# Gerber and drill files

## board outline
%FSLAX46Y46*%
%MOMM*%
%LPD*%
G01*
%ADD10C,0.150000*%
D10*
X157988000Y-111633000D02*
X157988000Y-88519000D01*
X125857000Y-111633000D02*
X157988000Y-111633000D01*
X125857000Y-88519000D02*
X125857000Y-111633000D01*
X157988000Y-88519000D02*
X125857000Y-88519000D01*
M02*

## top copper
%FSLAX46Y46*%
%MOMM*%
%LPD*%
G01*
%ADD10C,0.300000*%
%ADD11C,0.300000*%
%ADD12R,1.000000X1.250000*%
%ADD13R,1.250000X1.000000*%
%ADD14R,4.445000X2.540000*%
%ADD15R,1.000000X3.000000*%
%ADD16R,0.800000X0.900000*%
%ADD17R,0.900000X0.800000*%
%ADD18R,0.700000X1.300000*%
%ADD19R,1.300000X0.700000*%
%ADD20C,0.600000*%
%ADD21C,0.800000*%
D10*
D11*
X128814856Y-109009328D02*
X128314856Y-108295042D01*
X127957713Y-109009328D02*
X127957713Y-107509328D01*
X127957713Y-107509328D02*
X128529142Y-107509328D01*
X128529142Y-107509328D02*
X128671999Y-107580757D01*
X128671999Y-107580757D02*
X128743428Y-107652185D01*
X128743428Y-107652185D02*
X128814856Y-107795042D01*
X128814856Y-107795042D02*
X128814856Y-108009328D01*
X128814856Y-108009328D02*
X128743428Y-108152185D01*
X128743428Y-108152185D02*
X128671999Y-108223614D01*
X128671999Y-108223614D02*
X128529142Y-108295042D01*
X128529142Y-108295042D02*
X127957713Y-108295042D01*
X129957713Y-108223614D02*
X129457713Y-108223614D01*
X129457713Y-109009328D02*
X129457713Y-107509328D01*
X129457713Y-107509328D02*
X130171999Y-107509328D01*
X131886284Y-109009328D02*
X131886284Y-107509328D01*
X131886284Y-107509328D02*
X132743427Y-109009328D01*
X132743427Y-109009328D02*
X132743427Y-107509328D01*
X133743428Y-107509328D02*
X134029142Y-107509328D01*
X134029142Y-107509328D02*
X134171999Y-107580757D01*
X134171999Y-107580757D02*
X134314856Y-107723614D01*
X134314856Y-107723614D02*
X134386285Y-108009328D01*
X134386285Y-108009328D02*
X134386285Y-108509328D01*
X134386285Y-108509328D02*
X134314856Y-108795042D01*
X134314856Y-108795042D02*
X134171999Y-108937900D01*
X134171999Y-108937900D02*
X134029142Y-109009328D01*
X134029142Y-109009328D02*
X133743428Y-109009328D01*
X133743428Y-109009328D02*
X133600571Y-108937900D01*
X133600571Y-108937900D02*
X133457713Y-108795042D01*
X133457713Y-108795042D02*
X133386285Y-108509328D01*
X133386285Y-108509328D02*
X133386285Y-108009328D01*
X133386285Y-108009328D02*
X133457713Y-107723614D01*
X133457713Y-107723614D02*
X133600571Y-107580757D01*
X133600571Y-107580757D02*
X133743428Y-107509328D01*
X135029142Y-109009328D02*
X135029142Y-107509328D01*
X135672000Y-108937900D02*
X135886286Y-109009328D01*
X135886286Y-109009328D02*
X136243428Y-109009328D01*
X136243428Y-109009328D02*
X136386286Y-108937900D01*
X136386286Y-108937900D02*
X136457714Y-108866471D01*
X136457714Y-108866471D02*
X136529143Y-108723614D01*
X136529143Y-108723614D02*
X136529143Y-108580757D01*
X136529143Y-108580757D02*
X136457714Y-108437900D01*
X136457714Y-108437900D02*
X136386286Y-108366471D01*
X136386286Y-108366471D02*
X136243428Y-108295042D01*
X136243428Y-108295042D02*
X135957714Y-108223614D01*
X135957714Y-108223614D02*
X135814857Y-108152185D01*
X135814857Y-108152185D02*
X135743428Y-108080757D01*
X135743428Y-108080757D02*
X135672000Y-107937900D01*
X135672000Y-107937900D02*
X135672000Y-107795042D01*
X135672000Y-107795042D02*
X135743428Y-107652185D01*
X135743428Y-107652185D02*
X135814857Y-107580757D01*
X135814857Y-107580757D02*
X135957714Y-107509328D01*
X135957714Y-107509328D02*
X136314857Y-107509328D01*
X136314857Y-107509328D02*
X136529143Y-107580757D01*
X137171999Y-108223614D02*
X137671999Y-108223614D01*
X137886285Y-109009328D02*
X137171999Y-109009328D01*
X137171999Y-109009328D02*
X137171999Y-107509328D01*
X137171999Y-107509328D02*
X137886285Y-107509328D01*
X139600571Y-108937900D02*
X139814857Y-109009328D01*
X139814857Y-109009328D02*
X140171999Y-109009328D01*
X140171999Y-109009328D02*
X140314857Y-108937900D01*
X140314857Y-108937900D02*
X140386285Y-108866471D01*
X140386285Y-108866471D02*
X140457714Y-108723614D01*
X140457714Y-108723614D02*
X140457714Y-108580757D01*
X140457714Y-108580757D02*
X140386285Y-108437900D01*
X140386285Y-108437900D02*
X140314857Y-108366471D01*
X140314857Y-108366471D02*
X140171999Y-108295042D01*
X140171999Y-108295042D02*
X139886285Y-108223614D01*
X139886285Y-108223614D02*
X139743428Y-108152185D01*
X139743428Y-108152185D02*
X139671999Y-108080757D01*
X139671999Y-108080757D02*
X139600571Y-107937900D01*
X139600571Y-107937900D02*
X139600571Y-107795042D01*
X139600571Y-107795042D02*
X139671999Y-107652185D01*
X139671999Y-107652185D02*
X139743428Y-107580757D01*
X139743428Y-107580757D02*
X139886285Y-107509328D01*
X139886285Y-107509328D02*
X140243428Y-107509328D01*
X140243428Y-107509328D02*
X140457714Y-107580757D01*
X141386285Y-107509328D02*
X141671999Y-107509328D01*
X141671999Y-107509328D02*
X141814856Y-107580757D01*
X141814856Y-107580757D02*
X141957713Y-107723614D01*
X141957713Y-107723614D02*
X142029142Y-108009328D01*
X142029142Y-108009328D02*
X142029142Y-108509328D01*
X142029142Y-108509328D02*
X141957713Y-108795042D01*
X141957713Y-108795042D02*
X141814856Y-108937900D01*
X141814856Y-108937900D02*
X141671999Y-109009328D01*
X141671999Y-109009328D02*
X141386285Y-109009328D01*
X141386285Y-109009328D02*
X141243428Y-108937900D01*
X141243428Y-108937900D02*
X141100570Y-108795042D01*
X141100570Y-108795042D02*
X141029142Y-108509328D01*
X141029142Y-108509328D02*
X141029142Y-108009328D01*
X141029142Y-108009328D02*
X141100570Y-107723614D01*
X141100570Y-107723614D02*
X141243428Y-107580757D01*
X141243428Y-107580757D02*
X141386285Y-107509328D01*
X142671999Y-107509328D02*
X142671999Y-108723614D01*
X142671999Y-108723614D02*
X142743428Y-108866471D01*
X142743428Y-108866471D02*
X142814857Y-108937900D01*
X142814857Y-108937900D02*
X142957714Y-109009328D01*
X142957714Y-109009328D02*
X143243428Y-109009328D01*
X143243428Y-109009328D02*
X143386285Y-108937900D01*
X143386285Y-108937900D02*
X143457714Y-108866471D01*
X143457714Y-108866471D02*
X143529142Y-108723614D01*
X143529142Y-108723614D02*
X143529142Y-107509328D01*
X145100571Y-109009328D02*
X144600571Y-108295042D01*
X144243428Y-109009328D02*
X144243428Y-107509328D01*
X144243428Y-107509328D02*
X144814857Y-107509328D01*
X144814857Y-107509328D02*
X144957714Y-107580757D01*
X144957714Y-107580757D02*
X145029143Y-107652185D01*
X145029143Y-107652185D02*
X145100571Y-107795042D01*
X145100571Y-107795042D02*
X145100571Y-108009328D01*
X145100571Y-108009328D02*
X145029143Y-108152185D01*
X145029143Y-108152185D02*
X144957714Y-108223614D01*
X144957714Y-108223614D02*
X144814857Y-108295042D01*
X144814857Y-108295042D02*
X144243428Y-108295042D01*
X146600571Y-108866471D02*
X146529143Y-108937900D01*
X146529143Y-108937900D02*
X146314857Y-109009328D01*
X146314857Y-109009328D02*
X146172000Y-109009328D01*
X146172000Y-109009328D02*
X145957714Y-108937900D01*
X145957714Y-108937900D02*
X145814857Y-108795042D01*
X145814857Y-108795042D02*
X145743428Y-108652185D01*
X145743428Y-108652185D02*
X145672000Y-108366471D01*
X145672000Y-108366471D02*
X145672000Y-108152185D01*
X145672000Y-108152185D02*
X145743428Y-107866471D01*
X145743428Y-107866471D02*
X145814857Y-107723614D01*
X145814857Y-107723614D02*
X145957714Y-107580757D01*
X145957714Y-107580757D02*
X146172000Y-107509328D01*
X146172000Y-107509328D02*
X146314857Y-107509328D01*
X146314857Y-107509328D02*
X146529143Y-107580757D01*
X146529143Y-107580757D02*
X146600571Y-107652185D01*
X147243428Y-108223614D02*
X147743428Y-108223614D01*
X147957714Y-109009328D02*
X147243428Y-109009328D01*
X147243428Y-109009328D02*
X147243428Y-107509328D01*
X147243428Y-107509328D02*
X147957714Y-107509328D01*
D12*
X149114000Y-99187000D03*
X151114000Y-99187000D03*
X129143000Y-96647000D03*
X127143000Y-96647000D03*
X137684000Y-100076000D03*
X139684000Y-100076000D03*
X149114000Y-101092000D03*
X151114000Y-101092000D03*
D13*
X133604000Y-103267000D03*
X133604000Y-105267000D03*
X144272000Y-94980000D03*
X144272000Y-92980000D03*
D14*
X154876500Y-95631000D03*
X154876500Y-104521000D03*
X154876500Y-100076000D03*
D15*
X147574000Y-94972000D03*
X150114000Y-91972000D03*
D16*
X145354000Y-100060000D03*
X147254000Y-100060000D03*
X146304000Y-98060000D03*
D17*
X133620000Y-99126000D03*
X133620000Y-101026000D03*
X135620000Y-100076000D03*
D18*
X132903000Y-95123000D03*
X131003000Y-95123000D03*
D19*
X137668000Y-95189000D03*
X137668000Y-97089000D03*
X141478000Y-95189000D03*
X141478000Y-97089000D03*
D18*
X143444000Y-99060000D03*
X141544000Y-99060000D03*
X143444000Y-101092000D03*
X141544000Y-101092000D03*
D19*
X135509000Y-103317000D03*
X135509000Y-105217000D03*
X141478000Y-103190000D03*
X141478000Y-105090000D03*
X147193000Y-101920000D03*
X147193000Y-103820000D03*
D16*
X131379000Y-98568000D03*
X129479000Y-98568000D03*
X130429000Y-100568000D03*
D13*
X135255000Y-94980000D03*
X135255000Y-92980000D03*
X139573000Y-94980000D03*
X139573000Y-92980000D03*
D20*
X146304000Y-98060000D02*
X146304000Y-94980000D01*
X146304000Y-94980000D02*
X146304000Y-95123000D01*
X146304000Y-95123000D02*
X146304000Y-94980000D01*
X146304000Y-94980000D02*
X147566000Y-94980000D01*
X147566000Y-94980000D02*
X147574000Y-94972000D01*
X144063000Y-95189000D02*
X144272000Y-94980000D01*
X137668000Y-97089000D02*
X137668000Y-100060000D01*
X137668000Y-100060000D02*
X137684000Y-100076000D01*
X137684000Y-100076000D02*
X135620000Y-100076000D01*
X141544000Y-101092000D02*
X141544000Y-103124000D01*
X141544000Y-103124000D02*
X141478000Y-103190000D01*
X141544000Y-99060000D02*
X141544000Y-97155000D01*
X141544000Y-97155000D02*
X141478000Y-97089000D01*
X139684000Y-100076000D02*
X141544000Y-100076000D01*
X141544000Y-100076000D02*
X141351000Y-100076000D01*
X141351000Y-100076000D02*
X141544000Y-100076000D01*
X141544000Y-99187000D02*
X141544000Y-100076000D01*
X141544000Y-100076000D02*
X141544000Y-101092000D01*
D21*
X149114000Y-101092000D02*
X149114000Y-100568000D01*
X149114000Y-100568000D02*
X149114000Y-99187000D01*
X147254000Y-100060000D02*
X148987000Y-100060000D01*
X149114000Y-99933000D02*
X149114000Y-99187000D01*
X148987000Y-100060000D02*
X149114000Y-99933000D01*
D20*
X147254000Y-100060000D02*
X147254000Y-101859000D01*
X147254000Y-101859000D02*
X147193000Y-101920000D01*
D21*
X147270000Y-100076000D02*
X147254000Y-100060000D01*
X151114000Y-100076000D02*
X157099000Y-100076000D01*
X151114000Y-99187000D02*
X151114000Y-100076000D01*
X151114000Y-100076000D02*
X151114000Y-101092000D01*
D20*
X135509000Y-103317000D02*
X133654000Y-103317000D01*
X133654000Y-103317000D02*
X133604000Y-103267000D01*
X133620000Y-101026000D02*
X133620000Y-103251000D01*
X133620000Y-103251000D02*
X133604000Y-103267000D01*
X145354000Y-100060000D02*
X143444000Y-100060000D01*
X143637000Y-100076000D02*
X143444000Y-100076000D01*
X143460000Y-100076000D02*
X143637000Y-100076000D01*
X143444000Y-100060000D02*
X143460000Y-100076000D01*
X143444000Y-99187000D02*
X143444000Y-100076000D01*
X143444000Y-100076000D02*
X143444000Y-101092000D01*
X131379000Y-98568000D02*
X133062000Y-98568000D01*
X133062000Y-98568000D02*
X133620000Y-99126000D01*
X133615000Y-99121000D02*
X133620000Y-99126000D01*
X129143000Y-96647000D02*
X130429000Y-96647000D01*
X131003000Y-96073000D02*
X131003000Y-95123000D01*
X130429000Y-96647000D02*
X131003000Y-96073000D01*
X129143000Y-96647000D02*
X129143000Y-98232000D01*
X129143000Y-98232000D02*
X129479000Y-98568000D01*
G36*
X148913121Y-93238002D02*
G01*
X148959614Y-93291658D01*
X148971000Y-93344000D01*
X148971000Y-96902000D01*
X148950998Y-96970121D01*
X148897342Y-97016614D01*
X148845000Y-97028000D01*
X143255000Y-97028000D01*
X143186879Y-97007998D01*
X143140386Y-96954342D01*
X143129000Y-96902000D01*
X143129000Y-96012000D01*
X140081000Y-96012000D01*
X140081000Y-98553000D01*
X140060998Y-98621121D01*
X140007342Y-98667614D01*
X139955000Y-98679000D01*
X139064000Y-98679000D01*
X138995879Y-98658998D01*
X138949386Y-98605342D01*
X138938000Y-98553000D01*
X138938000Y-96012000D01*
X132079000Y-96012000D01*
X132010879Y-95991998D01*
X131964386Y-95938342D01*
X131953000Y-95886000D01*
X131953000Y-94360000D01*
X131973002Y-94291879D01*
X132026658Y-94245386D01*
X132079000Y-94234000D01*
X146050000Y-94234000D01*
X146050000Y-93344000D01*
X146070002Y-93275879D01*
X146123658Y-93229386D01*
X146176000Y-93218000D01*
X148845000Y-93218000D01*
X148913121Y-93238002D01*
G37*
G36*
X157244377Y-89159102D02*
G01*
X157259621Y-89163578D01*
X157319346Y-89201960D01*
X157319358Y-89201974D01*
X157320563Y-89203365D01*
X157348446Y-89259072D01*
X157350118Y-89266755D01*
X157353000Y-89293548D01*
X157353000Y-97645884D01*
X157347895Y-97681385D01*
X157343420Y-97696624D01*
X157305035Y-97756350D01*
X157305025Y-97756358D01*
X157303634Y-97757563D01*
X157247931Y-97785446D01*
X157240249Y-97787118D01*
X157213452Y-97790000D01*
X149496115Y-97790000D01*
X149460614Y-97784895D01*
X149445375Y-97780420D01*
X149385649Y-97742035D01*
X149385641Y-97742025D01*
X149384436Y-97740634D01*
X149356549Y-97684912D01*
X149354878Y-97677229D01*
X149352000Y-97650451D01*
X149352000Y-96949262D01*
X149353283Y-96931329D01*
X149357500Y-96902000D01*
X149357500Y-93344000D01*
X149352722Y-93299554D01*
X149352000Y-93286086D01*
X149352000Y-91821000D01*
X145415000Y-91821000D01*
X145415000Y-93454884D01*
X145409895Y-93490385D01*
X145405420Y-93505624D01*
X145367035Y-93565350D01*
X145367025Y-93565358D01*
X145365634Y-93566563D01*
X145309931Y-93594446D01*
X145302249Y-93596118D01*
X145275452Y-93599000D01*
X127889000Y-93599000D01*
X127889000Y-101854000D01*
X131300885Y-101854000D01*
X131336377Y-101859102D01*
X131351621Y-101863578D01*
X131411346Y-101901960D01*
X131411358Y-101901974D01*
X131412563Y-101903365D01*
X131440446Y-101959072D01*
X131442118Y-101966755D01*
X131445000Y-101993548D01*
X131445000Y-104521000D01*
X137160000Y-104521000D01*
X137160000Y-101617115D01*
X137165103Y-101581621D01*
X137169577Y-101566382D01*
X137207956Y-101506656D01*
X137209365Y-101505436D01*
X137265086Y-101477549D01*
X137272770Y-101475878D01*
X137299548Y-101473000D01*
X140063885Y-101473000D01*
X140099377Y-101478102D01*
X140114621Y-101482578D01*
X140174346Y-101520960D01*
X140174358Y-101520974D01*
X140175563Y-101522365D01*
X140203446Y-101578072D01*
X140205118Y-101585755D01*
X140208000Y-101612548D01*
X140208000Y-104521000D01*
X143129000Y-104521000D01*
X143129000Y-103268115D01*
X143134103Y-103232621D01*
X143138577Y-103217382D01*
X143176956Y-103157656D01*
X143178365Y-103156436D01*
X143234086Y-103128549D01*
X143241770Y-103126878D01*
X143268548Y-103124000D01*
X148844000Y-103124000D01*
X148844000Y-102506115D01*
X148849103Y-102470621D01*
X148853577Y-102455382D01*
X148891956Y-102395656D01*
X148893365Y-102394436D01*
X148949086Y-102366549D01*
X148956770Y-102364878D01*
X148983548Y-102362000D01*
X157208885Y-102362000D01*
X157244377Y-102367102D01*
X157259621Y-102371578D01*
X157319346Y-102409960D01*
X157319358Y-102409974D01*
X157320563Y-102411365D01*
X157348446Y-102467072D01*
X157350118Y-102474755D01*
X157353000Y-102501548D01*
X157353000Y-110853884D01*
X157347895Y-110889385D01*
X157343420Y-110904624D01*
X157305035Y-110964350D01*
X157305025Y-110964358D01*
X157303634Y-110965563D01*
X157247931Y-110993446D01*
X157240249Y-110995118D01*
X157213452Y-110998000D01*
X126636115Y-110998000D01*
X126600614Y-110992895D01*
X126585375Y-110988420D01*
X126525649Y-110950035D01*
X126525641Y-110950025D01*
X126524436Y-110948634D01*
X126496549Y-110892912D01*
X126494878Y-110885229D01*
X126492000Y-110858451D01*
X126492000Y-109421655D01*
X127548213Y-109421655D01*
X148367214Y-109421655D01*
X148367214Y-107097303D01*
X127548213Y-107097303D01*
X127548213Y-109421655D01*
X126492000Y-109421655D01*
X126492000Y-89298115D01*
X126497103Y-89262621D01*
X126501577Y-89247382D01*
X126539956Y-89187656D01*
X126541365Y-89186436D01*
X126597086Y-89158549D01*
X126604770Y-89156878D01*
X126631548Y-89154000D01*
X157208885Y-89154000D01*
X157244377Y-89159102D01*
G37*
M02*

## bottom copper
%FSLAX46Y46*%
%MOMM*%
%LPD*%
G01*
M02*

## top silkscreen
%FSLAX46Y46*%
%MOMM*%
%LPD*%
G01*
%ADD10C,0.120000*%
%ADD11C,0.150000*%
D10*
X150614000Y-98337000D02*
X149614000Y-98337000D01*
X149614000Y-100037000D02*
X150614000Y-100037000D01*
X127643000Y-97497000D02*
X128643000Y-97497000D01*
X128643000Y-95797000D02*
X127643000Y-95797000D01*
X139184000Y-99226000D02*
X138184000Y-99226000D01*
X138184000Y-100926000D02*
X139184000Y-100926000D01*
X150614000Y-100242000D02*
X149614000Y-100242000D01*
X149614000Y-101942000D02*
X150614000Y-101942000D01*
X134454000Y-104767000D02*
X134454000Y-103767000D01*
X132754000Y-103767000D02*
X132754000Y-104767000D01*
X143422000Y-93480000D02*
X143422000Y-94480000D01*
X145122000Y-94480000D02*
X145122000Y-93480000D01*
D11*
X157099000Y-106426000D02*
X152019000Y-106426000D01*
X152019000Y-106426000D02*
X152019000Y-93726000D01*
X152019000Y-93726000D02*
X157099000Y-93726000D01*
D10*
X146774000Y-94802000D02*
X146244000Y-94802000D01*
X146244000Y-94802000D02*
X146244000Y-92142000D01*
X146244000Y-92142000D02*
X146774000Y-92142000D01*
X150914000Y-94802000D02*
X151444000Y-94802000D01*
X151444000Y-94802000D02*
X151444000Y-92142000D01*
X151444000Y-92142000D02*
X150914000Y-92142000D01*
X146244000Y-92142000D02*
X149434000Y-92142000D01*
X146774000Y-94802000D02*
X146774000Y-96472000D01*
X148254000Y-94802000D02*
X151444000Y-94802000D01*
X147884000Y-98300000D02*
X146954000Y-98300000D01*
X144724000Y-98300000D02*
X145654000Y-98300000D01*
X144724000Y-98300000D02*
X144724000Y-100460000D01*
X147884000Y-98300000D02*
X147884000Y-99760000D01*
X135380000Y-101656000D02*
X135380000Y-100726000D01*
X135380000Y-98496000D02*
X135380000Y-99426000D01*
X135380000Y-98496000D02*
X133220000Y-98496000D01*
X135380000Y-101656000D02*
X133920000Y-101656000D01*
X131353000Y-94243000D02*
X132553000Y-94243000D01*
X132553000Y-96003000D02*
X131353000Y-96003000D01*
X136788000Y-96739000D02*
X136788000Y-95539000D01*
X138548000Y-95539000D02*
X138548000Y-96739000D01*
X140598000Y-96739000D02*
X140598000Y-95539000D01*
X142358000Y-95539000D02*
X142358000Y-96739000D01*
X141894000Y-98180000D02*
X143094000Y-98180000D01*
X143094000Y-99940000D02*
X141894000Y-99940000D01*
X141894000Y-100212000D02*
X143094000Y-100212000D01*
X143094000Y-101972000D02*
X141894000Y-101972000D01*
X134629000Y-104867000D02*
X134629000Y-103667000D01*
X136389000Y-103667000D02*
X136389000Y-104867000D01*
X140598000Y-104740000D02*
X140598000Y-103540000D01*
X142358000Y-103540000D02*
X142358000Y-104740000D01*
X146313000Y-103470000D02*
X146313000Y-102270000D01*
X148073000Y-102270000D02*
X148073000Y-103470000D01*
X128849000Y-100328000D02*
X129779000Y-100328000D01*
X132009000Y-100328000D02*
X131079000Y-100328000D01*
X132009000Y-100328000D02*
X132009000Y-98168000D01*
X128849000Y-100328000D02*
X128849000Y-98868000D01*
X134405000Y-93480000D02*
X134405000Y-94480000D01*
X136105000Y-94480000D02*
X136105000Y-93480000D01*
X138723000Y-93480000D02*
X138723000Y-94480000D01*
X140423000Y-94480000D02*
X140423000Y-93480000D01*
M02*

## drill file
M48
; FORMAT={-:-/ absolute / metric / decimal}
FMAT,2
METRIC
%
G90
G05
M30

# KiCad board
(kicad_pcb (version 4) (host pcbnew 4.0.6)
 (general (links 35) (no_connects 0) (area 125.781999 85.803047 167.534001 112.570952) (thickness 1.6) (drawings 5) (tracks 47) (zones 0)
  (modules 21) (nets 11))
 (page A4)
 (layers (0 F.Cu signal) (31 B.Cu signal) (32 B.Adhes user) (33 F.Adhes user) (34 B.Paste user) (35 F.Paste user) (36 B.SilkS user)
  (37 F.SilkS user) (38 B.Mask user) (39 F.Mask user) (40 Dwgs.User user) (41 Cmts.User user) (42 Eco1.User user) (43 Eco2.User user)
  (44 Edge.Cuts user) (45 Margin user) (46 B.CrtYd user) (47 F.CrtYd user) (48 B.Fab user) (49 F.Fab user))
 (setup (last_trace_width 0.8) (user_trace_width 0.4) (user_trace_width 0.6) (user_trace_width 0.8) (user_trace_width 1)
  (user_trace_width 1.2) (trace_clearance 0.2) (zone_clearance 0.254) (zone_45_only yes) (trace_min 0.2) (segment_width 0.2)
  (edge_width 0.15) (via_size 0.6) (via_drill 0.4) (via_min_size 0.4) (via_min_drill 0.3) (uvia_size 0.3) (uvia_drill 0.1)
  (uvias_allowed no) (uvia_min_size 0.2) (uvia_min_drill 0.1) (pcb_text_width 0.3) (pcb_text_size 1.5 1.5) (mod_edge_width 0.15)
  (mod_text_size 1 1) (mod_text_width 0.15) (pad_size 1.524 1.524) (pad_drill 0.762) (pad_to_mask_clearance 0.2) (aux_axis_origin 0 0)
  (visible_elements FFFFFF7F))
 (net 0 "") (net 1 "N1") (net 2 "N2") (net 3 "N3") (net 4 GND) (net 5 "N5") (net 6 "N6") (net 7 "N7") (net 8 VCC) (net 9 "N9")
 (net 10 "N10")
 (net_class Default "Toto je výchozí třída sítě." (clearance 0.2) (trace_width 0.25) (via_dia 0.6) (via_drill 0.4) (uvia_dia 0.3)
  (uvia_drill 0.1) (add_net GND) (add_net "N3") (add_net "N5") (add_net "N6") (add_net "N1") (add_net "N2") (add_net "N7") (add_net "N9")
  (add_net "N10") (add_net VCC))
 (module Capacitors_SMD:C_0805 (layer F.Cu) (at 150.114 99.187)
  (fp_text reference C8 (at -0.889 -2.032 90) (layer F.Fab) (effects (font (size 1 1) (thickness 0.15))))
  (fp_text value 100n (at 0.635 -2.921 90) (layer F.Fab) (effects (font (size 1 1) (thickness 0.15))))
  (fp_line (start 0.5 -0.85) (end -0.5 -0.85) (layer F.SilkS) (width 0.12))
  (fp_line (start -0.5 0.85) (end 0.5 0.85) (layer F.SilkS) (width 0.12))
  (pad 1 smd rect (at -1 0) (size 1 1.25) (layers F.Cu F.Paste F.Mask) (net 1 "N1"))
  (pad 2 smd rect (at 1 0) (size 1 1.25) (layers F.Cu F.Paste F.Mask) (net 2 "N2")))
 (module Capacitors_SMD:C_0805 (layer F.Cu) (at 128.143 96.647 180)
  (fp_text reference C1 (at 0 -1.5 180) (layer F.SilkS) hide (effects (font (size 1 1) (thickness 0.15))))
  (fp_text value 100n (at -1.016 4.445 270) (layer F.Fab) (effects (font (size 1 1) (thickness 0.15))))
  (fp_line (start 0.5 -0.85) (end -0.5 -0.85) (layer F.SilkS) (width 0.12))
  (fp_line (start -0.5 0.85) (end 0.5 0.85) (layer F.SilkS) (width 0.12))
  (pad 1 smd rect (at -1 0 180) (size 1 1.25) (layers F.Cu F.Paste F.Mask) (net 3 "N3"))
  (pad 2 smd rect (at 1 0 180) (size 1 1.25) (layers F.Cu F.Paste F.Mask) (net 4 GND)))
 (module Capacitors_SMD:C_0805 (layer F.Cu) (at 138.684 100.076)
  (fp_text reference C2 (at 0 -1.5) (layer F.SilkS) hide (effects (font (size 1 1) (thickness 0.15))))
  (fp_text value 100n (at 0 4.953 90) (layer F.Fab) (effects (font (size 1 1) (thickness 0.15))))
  (fp_line (start 0.5 -0.85) (end -0.5 -0.85) (layer F.SilkS) (width 0.12))
  (fp_line (start -0.5 0.85) (end 0.5 0.85) (layer F.SilkS) (width 0.12))
  (pad 1 smd rect (at -1 0) (size 1 1.25) (layers F.Cu F.Paste F.Mask) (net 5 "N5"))
  (pad 2 smd rect (at 1 0) (size 1 1.25) (layers F.Cu F.Paste F.Mask) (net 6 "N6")))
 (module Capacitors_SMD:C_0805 (layer F.Cu) (at 150.114 101.092)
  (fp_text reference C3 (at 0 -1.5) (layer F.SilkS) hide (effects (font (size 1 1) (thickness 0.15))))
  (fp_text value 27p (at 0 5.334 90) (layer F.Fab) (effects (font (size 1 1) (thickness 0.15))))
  (fp_line (start 0.5 -0.85) (end -0.5 -0.85) (layer F.SilkS) (width 0.12))
  (fp_line (start -0.5 0.85) (end 0.5 0.85) (layer F.SilkS) (width 0.12))
  (pad 1 smd rect (at -1 0) (size 1 1.25) (layers F.Cu F.Paste F.Mask) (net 1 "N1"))
  (pad 2 smd rect (at 1 0) (size 1 1.25) (layers F.Cu F.Paste F.Mask) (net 2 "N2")))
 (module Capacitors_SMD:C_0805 (layer F.Cu) (at 133.604 104.267 270)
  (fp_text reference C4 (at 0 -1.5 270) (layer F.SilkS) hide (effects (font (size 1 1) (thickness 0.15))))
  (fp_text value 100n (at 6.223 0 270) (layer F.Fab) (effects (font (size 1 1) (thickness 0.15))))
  (fp_line (start 0.5 -0.85) (end -0.5 -0.85) (layer F.SilkS) (width 0.12))
  (fp_line (start -0.5 0.85) (end 0.5 0.85) (layer F.SilkS) (width 0.12))
  (pad 1 smd rect (at -1 0 270) (size 1 1.25) (layers F.Cu F.Paste F.Mask) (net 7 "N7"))
  (pad 2 smd rect (at 1 0 270) (size 1 1.25) (layers F.Cu F.Paste F.Mask) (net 4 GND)))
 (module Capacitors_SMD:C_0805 (layer F.Cu) (at 144.272 93.98 90)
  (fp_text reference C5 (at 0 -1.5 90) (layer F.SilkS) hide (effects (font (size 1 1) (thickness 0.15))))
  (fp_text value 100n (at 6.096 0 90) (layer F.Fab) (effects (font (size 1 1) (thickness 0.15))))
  (fp_line (start 0.5 -0.85) (end -0.5 -0.85) (layer F.SilkS) (width 0.12))
  (fp_line (start -0.5 0.85) (end 0.5 0.85) (layer F.SilkS) (width 0.12))
  (pad 1 smd rect (at -1 0 90) (size 1 1.25) (layers F.Cu F.Paste F.Mask) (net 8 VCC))
  (pad 2 smd rect (at 1 0 90) (size 1 1.25) (layers F.Cu F.Paste F.Mask) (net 4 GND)))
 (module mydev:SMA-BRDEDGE (layer F.Cu) (at 157.099 100.076 180)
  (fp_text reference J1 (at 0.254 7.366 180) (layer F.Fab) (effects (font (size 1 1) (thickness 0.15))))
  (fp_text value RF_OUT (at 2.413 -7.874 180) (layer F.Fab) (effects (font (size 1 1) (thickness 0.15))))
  (fp_line (start 0 -6.35) (end 5.08 -6.35) (layer F.SilkS) (width 0.15))
  (fp_line (start 5.08 -6.35) (end 5.08 6.35) (layer F.SilkS) (width 0.15))
  (fp_line (start 5.08 6.35) (end 0 6.35) (layer F.SilkS) (width 0.15))
  (pad 2 smd rect (at 0 4.445 180) (size 4.445 2.54) (drill (offset 2.2225 0)) (layers F.Cu F.Paste F.Mask) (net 4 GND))
  (pad 2 smd rect (at 0 -4.445 180) (size 4.445 2.54) (drill (offset 2.2225 0)) (layers F.Cu F.Paste F.Mask) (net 4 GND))
  (pad 1 smd rect (at 0 0 180) (size 4.445 2.54) (drill (offset 2.2225 0)) (layers F.Cu F.Paste F.Mask) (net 2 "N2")))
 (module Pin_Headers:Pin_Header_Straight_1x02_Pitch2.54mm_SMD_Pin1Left (layer F.Cu) (at 148.844 93.472 90)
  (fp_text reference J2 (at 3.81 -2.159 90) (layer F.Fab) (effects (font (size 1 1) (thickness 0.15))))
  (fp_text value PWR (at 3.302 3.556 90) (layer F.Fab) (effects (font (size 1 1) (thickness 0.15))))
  (fp_line (start -1.33 -2.07) (end -1.33 -2.6) (layer F.SilkS) (width 0.12))
  (fp_line (start -1.33 -2.6) (end 1.33 -2.6) (layer F.SilkS) (width 0.12))
  (fp_line (start 1.33 -2.6) (end 1.33 -2.07) (layer F.SilkS) (width 0.12))
  (fp_line (start -1.33 2.07) (end -1.33 2.6) (layer F.SilkS) (width 0.12))
  (fp_line (start -1.33 2.6) (end 1.33 2.6) (layer F.SilkS) (width 0.12))
  (fp_line (start 1.33 2.6) (end 1.33 2.07) (layer F.SilkS) (width 0.12))
  (fp_line (start 1.33 -2.6) (end 1.33 0.59) (layer F.SilkS) (width 0.12))
  (fp_line (start -1.33 -2.07) (end -3 -2.07) (layer F.SilkS) (width 0.12))
  (fp_line (start -1.33 -0.59) (end -1.33 2.6) (layer F.SilkS) (width 0.12))
  (pad 1 smd rect (at -1.5 -1.27 90) (size 3 1) (layers F.Cu F.Mask) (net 8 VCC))
  (pad 2 smd rect (at 1.5 1.27 90) (size 3 1) (layers F.Cu F.Mask) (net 4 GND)))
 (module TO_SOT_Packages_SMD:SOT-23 (layer F.Cu) (at 146.304 99.06 90)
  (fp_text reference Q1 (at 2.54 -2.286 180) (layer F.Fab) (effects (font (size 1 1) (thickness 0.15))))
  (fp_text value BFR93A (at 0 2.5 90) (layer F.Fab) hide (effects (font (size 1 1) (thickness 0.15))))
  (fp_line (start 0.76 1.58) (end 0.76 0.65) (layer F.SilkS) (width 0.12))
  (fp_line (start 0.76 -1.58) (end 0.76 -0.65) (layer F.SilkS) (width 0.12))
  (fp_line (start 0.76 -1.58) (end -1.4 -1.58) (layer F.SilkS) (width 0.12))
  (fp_line (start 0.76 1.58) (end -0.7 1.58) (layer F.SilkS) (width 0.12))
  (pad 1 smd rect (at -1 -0.95 90) (size 0.9 0.8) (layers F.Cu F.Paste F.Mask) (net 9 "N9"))
  (pad 2 smd rect (at -1 0.95 90) (size 0.9 0.8) (layers F.Cu F.Paste F.Mask) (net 1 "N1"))
  (pad 3 smd rect (at 1 0 90) (size 0.9 0.8) (layers F.Cu F.Paste F.Mask) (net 8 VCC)))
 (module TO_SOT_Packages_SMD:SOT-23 (layer F.Cu) (at 134.62 100.076)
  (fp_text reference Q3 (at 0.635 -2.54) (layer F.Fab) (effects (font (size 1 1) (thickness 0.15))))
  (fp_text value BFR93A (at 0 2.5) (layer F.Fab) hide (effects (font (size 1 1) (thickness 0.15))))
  (fp_line (start 0.76 1.58) (end 0.76 0.65) (layer F.SilkS) (width 0.12))
  (fp_line (start 0.76 -1.58) (end 0.76 -0.65) (layer F.SilkS) (width 0.12))
  (fp_line (start 0.76 -1.58) (end -1.4 -1.58) (layer F.SilkS) (width 0.12))
  (fp_line (start 0.76 1.58) (end -0.7 1.58) (layer F.SilkS) (width 0.12))
  (pad 1 smd rect (at -1 -0.95) (size 0.9 0.8) (layers F.Cu F.Paste F.Mask) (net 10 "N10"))
  (pad 2 smd rect (at -1 0.95) (size 0.9 0.8) (layers F.Cu F.Paste F.Mask) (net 7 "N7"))
  (pad 3 smd rect (at 1 0) (size 0.9 0.8) (layers F.Cu F.Paste F.Mask) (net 5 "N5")))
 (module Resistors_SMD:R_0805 (layer F.Cu) (at 131.953 95.123 180)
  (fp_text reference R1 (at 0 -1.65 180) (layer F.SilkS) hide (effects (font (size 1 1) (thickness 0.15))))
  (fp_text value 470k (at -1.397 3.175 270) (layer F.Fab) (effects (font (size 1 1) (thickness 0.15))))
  (fp_line (start 0.6 0.88) (end -0.6 0.88) (layer F.SilkS) (width 0.12))
  (fp_line (start -0.6 -0.88) (end 0.6 -0.88) (layer F.SilkS) (width 0.12))
  (pad 1 smd rect (at -0.95 0 180) (size 0.7 1.3) (layers F.Cu F.Paste F.Mask) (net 8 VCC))
  (pad 2 smd rect (at 0.95 0 180) (size 0.7 1.3) (layers F.Cu F.Paste F.Mask) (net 3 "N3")))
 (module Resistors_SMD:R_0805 (layer F.Cu) (at 137.668 96.139 270)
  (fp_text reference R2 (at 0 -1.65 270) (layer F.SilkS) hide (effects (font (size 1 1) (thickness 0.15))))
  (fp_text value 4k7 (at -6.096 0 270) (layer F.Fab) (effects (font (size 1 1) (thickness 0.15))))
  (fp_line (start 0.6 0.88) (end -0.6 0.88) (layer F.SilkS) (width 0.12))
  (fp_line (start -0.6 -0.88) (end 0.6 -0.88) (layer F.SilkS) (width 0.12))
  (pad 1 smd rect (at -0.95 0 270) (size 0.7 1.3) (layers F.Cu F.Paste F.Mask) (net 8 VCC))
  (pad 2 smd rect (at 0.95 0 270) (size 0.7 1.3) (layers F.Cu F.Paste F.Mask) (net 5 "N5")))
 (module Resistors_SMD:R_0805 (layer F.Cu) (at 141.478 96.139 270)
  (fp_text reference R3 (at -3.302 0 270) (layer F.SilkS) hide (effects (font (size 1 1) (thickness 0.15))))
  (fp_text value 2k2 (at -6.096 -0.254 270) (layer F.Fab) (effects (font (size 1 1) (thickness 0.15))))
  (fp_line (start 0.6 0.88) (end -0.6 0.88) (layer F.SilkS) (width 0.12))
  (fp_line (start -0.6 -0.88) (end 0.6 -0.88) (layer F.SilkS) (width 0.12))
  (pad 1 smd rect (at -0.95 0 270) (size 0.7 1.3) (layers F.Cu F.Paste F.Mask) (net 8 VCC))
  (pad 2 smd rect (at 0.95 0 270) (size 0.7 1.3) (layers F.Cu F.Paste F.Mask) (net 6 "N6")))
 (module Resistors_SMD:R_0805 (layer F.Cu) (at 142.494 99.06 180)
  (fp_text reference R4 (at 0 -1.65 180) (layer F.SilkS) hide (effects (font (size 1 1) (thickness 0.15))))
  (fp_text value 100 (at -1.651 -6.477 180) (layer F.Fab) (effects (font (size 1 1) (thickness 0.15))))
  (fp_line (start 0.6 0.88) (end -0.6 0.88) (layer F.SilkS) (width 0.12))
  (fp_line (start -0.6 -0.88) (end 0.6 -0.88) (layer F.SilkS) (width 0.12))
  (pad 1 smd rect (at -0.95 0 180) (size 0.7 1.3) (layers F.Cu F.Paste F.Mask) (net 9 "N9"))
  (pad 2 smd rect (at 0.95 0 180) (size 0.7 1.3) (layers F.Cu F.Paste F.Mask) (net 6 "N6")))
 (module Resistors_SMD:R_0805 (layer F.Cu) (at 142.494 101.092 180)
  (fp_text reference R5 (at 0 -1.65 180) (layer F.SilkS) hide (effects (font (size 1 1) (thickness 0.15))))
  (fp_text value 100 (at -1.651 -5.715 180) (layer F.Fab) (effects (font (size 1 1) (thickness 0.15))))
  (fp_line (start 0.6 0.88) (end -0.6 0.88) (layer F.SilkS) (width 0.12))
  (fp_line (start -0.6 -0.88) (end 0.6 -0.88) (layer F.SilkS) (width 0.12))
  (pad 1 smd rect (at -0.95 0 180) (size 0.7 1.3) (layers F.Cu F.Paste F.Mask) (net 9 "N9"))
  (pad 2 smd rect (at 0.95 0 180) (size 0.7 1.3) (layers F.Cu F.Paste F.Mask) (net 6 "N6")))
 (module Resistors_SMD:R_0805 (layer F.Cu) (at 135.509 104.267 270)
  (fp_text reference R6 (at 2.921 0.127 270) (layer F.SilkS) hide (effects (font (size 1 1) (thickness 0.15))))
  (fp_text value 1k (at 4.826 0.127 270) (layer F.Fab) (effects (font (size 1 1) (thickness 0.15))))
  (fp_line (start 0.6 0.88) (end -0.6 0.88) (layer F.SilkS) (width 0.12))
  (fp_line (start -0.6 -0.88) (end 0.6 -0.88) (layer F.SilkS) (width 0.12))
  (pad 1 smd rect (at -0.95 0 270) (size 0.7 1.3) (layers F.Cu F.Paste F.Mask) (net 7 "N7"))
  (pad 2 smd rect (at 0.95 0 270) (size 0.7 1.3) (layers F.Cu F.Paste F.Mask) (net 4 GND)))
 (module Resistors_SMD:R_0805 (layer F.Cu) (at 141.478 104.14 270)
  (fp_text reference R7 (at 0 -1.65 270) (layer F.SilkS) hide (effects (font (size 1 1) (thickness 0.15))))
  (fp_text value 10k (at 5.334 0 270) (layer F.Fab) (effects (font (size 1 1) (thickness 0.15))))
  (fp_line (start 0.6 0.88) (end -0.6 0.88) (layer F.SilkS) (width 0.12))
  (fp_line (start -0.6 -0.88) (end 0.6 -0.88) (layer F.SilkS) (width 0.12))
  (pad 1 smd rect (at -0.95 0 270) (size 0.7 1.3) (layers F.Cu F.Paste F.Mask) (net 6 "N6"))
  (pad 2 smd rect (at 0.95 0 270) (size 0.7 1.3) (layers F.Cu F.Paste F.Mask) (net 4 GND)))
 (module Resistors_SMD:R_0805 (layer F.Cu) (at 147.193 102.87 270)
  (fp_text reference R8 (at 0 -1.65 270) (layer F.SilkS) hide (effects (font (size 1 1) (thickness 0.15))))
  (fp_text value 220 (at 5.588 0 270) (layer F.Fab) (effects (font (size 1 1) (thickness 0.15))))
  (fp_line (start 0.6 0.88) (end -0.6 0.88) (layer F.SilkS) (width 0.12))
  (fp_line (start -0.6 -0.88) (end 0.6 -0.88) (layer F.SilkS) (width 0.12))
  (pad 1 smd rect (at -0.95 0 270) (size 0.7 1.3) (layers F.Cu F.Paste F.Mask) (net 1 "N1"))
  (pad 2 smd rect (at 0.95 0 270) (size 0.7 1.3) (layers F.Cu F.Paste F.Mask) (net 4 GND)))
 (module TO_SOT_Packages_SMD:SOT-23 (layer F.Cu) (at 130.429 99.568 270)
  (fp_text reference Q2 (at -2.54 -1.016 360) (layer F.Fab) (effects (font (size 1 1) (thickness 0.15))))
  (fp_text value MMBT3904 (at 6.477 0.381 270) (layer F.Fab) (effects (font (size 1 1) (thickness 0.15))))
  (fp_line (start 0.76 1.58) (end 0.76 0.65) (layer F.SilkS) (width 0.12))
  (fp_line (start 0.76 -1.58) (end 0.76 -0.65) (layer F.SilkS) (width 0.12))
  (fp_line (start 0.76 -1.58) (end -1.4 -1.58) (layer F.SilkS) (width 0.12))
  (fp_line (start 0.76 1.58) (end -0.7 1.58) (layer F.SilkS) (width 0.12))
  (pad 1 smd rect (at -1 -0.95 270) (size 0.9 0.8) (layers F.Cu F.Paste F.Mask) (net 10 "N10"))
  (pad 2 smd rect (at -1 0.95 270) (size 0.9 0.8) (layers F.Cu F.Paste F.Mask) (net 3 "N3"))
  (pad 3 smd rect (at 1 0 270) (size 0.9 0.8) (layers F.Cu F.Paste F.Mask)))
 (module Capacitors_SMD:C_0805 (layer F.Cu) (at 135.255 93.98 90)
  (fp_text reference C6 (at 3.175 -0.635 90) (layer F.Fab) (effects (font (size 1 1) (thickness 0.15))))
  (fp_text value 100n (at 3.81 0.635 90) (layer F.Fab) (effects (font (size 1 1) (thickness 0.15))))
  (fp_line (start 0.5 -0.85) (end -0.5 -0.85) (layer F.SilkS) (width 0.12))
  (fp_line (start -0.5 0.85) (end 0.5 0.85) (layer F.SilkS) (width 0.12))
  (pad 1 smd rect (at -1 0 90) (size 1 1.25) (layers F.Cu F.Paste F.Mask) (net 8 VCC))
  (pad 2 smd rect (at 1 0 90) (size 1 1.25) (layers F.Cu F.Paste F.Mask) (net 4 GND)))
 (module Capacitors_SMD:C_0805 (layer F.Cu) (at 139.573 93.98 90)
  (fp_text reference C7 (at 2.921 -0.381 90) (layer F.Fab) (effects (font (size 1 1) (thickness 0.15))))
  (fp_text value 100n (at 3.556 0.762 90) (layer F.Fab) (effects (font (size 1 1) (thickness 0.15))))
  (fp_line (start 0.5 -0.85) (end -0.5 -0.85) (layer F.SilkS) (width 0.12))
  (fp_line (start -0.5 0.85) (end 0.5 0.85) (layer F.SilkS) (width 0.12))
  (pad 1 smd rect (at -1 0 90) (size 1 1.25) (layers F.Cu F.Paste F.Mask) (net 8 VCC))
  (pad 2 smd rect (at 1 0 90) (size 1 1.25) (layers F.Cu F.Paste F.Mask) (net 4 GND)))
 (gr_line (start 157.988 111.633) (end 157.988 88.519) (angle 90) (layer Edge.Cuts) (width 0.15))
 (gr_line (start 125.857 111.633) (end 157.988 111.633) (angle 90) (layer Edge.Cuts) (width 0.15))
 (gr_line (start 125.857 88.519) (end 125.857 111.633) (angle 90) (layer Edge.Cuts) (width 0.15))
 (gr_line (start 157.988 88.519) (end 125.857 88.519) (angle 90) (layer Edge.Cuts) (width 0.15))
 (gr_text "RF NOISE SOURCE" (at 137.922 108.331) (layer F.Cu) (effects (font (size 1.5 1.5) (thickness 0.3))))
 (segment (start 146.304 98.06) (end 146.304 94.98) (width 0.6) (layer F.Cu) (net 8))
 (segment (start 146.304 94.98) (end 146.304 95.123) (width 0.6) (layer F.Cu) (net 8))
 (segment (start 146.304 95.123) (end 146.304 94.98) (width 0.6) (layer F.Cu) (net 8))
 (segment (start 146.304 94.98) (end 147.566 94.98) (width 0.6) (layer F.Cu) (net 8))
 (segment (start 147.566 94.98) (end 147.574 94.972) (width 0.6) (layer F.Cu) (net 8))
 (segment (start 144.063 95.189) (end 144.272 94.98) (width 0.6) (layer F.Cu) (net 8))
 (segment (start 137.668 97.089) (end 137.668 100.06) (width 0.6) (layer F.Cu) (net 5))
 (segment (start 137.668 100.06) (end 137.684 100.076) (width 0.6) (layer F.Cu) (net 5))
 (segment (start 137.684 100.076) (end 135.62 100.076) (width 0.6) (layer F.Cu) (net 5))
 (segment (start 141.544 101.092) (end 141.544 103.124) (width 0.6) (layer F.Cu) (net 6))
 (segment (start 141.544 103.124) (end 141.478 103.19) (width 0.6) (layer F.Cu) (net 6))
 (segment (start 141.544 99.06) (end 141.544 97.155) (width 0.6) (layer F.Cu) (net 6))
 (segment (start 141.544 97.155) (end 141.478 97.089) (width 0.6) (layer F.Cu) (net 6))
 (segment (start 139.684 100.076) (end 141.544 100.076) (width 0.6) (layer F.Cu) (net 6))
 (segment (start 141.544 100.076) (end 141.351 100.076) (width 0.6) (layer F.Cu) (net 6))
 (segment (start 141.351 100.076) (end 141.544 100.076) (width 0.6) (layer F.Cu) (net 6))
 (segment (start 141.544 99.187) (end 141.544 100.076) (width 0.6) (layer F.Cu) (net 6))
 (segment (start 141.544 100.076) (end 141.544 101.092) (width 0.6) (layer F.Cu) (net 6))
 (segment (start 149.114 101.092) (end 149.114 100.568) (width 0.8) (layer F.Cu) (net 1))
 (segment (start 149.114 100.568) (end 149.114 99.187) (width 0.8) (layer F.Cu) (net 1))
 (segment (start 147.254 100.06) (end 148.987 100.06) (width 0.8) (layer F.Cu) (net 1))
 (segment (start 149.114 99.933) (end 149.114 99.187) (width 0.8) (layer F.Cu) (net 1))
 (segment (start 148.987 100.06) (end 149.114 99.933) (width 0.8) (layer F.Cu) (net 1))
 (segment (start 147.254 100.06) (end 147.254 101.859) (width 0.6) (layer F.Cu) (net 1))
 (segment (start 147.254 101.859) (end 147.193 101.92) (width 0.6) (layer F.Cu) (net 1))
 (segment (start 147.27 100.076) (end 147.254 100.06) (width 0.8) (layer F.Cu) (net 1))
 (segment (start 151.114 100.076) (end 157.099 100.076) (width 0.8) (layer F.Cu) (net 2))
 (segment (start 151.114 99.187) (end 151.114 100.076) (width 0.8) (layer F.Cu) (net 2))
 (segment (start 151.114 100.076) (end 151.114 101.092) (width 0.8) (layer F.Cu) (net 2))
 (segment (start 135.509 103.317) (end 133.654 103.317) (width 0.6) (layer F.Cu) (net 7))
 (segment (start 133.654 103.317) (end 133.604 103.267) (width 0.6) (layer F.Cu) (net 7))
 (segment (start 133.62 101.026) (end 133.62 103.251) (width 0.6) (layer F.Cu) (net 7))
 (segment (start 133.62 103.251) (end 133.604 103.267) (width 0.6) (layer F.Cu) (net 7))
 (segment (start 145.354 100.06) (end 143.444 100.06) (width 0.6) (layer F.Cu) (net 9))
 (segment (start 143.637 100.076) (end 143.444 100.076) (width 0.6) (layer F.Cu) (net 9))
 (segment (start 143.46 100.076) (end 143.637 100.076) (width 0.6) (layer F.Cu) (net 9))
 (segment (start 143.444 100.06) (end 143.46 100.076) (width 0.6) (layer F.Cu) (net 9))
 (segment (start 143.444 99.187) (end 143.444 100.076) (width 0.6) (layer F.Cu) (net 9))
 (segment (start 143.444 100.076) (end 143.444 101.092) (width 0.6) (layer F.Cu) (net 9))
 (segment (start 131.379 98.568) (end 133.062 98.568) (width 0.6) (layer F.Cu) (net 10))
 (segment (start 133.062 98.568) (end 133.62 99.126) (width 0.6) (layer F.Cu) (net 10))
 (segment (start 133.615 99.121) (end 133.62 99.126) (width 0.6) (layer F.Cu) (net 10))
 (segment (start 129.143 96.647) (end 130.429 96.647) (width 0.6) (layer F.Cu) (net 3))
 (segment (start 131.003 96.073) (end 131.003 95.123) (width 0.6) (layer F.Cu) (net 3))
 (segment (start 130.429 96.647) (end 131.003 96.073) (width 0.6) (layer F.Cu) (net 3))
 (segment (start 129.143 96.647) (end 129.143 98.232) (width 0.6) (layer F.Cu) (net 3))
 (segment (start 129.143 98.232) (end 129.479 98.568) (width 0.6) (layer F.Cu) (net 3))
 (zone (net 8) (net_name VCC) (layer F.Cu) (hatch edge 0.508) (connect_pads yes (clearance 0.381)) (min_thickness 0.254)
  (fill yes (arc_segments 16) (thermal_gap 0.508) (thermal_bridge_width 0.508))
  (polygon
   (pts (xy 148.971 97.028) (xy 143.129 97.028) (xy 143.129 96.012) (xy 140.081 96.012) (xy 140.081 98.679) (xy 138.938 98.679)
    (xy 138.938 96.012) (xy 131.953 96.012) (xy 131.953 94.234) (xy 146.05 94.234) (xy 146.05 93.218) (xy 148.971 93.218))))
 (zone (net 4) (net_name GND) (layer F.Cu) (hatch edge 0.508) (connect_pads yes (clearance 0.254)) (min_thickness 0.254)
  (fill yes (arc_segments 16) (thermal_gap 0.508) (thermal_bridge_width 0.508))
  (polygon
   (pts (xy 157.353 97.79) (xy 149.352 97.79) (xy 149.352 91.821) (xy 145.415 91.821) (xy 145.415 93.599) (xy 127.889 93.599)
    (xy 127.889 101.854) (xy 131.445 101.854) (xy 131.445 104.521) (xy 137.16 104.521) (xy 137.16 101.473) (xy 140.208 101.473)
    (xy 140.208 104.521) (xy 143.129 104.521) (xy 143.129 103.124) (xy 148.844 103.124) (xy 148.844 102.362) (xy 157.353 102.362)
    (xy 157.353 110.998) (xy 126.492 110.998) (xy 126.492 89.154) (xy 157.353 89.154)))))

